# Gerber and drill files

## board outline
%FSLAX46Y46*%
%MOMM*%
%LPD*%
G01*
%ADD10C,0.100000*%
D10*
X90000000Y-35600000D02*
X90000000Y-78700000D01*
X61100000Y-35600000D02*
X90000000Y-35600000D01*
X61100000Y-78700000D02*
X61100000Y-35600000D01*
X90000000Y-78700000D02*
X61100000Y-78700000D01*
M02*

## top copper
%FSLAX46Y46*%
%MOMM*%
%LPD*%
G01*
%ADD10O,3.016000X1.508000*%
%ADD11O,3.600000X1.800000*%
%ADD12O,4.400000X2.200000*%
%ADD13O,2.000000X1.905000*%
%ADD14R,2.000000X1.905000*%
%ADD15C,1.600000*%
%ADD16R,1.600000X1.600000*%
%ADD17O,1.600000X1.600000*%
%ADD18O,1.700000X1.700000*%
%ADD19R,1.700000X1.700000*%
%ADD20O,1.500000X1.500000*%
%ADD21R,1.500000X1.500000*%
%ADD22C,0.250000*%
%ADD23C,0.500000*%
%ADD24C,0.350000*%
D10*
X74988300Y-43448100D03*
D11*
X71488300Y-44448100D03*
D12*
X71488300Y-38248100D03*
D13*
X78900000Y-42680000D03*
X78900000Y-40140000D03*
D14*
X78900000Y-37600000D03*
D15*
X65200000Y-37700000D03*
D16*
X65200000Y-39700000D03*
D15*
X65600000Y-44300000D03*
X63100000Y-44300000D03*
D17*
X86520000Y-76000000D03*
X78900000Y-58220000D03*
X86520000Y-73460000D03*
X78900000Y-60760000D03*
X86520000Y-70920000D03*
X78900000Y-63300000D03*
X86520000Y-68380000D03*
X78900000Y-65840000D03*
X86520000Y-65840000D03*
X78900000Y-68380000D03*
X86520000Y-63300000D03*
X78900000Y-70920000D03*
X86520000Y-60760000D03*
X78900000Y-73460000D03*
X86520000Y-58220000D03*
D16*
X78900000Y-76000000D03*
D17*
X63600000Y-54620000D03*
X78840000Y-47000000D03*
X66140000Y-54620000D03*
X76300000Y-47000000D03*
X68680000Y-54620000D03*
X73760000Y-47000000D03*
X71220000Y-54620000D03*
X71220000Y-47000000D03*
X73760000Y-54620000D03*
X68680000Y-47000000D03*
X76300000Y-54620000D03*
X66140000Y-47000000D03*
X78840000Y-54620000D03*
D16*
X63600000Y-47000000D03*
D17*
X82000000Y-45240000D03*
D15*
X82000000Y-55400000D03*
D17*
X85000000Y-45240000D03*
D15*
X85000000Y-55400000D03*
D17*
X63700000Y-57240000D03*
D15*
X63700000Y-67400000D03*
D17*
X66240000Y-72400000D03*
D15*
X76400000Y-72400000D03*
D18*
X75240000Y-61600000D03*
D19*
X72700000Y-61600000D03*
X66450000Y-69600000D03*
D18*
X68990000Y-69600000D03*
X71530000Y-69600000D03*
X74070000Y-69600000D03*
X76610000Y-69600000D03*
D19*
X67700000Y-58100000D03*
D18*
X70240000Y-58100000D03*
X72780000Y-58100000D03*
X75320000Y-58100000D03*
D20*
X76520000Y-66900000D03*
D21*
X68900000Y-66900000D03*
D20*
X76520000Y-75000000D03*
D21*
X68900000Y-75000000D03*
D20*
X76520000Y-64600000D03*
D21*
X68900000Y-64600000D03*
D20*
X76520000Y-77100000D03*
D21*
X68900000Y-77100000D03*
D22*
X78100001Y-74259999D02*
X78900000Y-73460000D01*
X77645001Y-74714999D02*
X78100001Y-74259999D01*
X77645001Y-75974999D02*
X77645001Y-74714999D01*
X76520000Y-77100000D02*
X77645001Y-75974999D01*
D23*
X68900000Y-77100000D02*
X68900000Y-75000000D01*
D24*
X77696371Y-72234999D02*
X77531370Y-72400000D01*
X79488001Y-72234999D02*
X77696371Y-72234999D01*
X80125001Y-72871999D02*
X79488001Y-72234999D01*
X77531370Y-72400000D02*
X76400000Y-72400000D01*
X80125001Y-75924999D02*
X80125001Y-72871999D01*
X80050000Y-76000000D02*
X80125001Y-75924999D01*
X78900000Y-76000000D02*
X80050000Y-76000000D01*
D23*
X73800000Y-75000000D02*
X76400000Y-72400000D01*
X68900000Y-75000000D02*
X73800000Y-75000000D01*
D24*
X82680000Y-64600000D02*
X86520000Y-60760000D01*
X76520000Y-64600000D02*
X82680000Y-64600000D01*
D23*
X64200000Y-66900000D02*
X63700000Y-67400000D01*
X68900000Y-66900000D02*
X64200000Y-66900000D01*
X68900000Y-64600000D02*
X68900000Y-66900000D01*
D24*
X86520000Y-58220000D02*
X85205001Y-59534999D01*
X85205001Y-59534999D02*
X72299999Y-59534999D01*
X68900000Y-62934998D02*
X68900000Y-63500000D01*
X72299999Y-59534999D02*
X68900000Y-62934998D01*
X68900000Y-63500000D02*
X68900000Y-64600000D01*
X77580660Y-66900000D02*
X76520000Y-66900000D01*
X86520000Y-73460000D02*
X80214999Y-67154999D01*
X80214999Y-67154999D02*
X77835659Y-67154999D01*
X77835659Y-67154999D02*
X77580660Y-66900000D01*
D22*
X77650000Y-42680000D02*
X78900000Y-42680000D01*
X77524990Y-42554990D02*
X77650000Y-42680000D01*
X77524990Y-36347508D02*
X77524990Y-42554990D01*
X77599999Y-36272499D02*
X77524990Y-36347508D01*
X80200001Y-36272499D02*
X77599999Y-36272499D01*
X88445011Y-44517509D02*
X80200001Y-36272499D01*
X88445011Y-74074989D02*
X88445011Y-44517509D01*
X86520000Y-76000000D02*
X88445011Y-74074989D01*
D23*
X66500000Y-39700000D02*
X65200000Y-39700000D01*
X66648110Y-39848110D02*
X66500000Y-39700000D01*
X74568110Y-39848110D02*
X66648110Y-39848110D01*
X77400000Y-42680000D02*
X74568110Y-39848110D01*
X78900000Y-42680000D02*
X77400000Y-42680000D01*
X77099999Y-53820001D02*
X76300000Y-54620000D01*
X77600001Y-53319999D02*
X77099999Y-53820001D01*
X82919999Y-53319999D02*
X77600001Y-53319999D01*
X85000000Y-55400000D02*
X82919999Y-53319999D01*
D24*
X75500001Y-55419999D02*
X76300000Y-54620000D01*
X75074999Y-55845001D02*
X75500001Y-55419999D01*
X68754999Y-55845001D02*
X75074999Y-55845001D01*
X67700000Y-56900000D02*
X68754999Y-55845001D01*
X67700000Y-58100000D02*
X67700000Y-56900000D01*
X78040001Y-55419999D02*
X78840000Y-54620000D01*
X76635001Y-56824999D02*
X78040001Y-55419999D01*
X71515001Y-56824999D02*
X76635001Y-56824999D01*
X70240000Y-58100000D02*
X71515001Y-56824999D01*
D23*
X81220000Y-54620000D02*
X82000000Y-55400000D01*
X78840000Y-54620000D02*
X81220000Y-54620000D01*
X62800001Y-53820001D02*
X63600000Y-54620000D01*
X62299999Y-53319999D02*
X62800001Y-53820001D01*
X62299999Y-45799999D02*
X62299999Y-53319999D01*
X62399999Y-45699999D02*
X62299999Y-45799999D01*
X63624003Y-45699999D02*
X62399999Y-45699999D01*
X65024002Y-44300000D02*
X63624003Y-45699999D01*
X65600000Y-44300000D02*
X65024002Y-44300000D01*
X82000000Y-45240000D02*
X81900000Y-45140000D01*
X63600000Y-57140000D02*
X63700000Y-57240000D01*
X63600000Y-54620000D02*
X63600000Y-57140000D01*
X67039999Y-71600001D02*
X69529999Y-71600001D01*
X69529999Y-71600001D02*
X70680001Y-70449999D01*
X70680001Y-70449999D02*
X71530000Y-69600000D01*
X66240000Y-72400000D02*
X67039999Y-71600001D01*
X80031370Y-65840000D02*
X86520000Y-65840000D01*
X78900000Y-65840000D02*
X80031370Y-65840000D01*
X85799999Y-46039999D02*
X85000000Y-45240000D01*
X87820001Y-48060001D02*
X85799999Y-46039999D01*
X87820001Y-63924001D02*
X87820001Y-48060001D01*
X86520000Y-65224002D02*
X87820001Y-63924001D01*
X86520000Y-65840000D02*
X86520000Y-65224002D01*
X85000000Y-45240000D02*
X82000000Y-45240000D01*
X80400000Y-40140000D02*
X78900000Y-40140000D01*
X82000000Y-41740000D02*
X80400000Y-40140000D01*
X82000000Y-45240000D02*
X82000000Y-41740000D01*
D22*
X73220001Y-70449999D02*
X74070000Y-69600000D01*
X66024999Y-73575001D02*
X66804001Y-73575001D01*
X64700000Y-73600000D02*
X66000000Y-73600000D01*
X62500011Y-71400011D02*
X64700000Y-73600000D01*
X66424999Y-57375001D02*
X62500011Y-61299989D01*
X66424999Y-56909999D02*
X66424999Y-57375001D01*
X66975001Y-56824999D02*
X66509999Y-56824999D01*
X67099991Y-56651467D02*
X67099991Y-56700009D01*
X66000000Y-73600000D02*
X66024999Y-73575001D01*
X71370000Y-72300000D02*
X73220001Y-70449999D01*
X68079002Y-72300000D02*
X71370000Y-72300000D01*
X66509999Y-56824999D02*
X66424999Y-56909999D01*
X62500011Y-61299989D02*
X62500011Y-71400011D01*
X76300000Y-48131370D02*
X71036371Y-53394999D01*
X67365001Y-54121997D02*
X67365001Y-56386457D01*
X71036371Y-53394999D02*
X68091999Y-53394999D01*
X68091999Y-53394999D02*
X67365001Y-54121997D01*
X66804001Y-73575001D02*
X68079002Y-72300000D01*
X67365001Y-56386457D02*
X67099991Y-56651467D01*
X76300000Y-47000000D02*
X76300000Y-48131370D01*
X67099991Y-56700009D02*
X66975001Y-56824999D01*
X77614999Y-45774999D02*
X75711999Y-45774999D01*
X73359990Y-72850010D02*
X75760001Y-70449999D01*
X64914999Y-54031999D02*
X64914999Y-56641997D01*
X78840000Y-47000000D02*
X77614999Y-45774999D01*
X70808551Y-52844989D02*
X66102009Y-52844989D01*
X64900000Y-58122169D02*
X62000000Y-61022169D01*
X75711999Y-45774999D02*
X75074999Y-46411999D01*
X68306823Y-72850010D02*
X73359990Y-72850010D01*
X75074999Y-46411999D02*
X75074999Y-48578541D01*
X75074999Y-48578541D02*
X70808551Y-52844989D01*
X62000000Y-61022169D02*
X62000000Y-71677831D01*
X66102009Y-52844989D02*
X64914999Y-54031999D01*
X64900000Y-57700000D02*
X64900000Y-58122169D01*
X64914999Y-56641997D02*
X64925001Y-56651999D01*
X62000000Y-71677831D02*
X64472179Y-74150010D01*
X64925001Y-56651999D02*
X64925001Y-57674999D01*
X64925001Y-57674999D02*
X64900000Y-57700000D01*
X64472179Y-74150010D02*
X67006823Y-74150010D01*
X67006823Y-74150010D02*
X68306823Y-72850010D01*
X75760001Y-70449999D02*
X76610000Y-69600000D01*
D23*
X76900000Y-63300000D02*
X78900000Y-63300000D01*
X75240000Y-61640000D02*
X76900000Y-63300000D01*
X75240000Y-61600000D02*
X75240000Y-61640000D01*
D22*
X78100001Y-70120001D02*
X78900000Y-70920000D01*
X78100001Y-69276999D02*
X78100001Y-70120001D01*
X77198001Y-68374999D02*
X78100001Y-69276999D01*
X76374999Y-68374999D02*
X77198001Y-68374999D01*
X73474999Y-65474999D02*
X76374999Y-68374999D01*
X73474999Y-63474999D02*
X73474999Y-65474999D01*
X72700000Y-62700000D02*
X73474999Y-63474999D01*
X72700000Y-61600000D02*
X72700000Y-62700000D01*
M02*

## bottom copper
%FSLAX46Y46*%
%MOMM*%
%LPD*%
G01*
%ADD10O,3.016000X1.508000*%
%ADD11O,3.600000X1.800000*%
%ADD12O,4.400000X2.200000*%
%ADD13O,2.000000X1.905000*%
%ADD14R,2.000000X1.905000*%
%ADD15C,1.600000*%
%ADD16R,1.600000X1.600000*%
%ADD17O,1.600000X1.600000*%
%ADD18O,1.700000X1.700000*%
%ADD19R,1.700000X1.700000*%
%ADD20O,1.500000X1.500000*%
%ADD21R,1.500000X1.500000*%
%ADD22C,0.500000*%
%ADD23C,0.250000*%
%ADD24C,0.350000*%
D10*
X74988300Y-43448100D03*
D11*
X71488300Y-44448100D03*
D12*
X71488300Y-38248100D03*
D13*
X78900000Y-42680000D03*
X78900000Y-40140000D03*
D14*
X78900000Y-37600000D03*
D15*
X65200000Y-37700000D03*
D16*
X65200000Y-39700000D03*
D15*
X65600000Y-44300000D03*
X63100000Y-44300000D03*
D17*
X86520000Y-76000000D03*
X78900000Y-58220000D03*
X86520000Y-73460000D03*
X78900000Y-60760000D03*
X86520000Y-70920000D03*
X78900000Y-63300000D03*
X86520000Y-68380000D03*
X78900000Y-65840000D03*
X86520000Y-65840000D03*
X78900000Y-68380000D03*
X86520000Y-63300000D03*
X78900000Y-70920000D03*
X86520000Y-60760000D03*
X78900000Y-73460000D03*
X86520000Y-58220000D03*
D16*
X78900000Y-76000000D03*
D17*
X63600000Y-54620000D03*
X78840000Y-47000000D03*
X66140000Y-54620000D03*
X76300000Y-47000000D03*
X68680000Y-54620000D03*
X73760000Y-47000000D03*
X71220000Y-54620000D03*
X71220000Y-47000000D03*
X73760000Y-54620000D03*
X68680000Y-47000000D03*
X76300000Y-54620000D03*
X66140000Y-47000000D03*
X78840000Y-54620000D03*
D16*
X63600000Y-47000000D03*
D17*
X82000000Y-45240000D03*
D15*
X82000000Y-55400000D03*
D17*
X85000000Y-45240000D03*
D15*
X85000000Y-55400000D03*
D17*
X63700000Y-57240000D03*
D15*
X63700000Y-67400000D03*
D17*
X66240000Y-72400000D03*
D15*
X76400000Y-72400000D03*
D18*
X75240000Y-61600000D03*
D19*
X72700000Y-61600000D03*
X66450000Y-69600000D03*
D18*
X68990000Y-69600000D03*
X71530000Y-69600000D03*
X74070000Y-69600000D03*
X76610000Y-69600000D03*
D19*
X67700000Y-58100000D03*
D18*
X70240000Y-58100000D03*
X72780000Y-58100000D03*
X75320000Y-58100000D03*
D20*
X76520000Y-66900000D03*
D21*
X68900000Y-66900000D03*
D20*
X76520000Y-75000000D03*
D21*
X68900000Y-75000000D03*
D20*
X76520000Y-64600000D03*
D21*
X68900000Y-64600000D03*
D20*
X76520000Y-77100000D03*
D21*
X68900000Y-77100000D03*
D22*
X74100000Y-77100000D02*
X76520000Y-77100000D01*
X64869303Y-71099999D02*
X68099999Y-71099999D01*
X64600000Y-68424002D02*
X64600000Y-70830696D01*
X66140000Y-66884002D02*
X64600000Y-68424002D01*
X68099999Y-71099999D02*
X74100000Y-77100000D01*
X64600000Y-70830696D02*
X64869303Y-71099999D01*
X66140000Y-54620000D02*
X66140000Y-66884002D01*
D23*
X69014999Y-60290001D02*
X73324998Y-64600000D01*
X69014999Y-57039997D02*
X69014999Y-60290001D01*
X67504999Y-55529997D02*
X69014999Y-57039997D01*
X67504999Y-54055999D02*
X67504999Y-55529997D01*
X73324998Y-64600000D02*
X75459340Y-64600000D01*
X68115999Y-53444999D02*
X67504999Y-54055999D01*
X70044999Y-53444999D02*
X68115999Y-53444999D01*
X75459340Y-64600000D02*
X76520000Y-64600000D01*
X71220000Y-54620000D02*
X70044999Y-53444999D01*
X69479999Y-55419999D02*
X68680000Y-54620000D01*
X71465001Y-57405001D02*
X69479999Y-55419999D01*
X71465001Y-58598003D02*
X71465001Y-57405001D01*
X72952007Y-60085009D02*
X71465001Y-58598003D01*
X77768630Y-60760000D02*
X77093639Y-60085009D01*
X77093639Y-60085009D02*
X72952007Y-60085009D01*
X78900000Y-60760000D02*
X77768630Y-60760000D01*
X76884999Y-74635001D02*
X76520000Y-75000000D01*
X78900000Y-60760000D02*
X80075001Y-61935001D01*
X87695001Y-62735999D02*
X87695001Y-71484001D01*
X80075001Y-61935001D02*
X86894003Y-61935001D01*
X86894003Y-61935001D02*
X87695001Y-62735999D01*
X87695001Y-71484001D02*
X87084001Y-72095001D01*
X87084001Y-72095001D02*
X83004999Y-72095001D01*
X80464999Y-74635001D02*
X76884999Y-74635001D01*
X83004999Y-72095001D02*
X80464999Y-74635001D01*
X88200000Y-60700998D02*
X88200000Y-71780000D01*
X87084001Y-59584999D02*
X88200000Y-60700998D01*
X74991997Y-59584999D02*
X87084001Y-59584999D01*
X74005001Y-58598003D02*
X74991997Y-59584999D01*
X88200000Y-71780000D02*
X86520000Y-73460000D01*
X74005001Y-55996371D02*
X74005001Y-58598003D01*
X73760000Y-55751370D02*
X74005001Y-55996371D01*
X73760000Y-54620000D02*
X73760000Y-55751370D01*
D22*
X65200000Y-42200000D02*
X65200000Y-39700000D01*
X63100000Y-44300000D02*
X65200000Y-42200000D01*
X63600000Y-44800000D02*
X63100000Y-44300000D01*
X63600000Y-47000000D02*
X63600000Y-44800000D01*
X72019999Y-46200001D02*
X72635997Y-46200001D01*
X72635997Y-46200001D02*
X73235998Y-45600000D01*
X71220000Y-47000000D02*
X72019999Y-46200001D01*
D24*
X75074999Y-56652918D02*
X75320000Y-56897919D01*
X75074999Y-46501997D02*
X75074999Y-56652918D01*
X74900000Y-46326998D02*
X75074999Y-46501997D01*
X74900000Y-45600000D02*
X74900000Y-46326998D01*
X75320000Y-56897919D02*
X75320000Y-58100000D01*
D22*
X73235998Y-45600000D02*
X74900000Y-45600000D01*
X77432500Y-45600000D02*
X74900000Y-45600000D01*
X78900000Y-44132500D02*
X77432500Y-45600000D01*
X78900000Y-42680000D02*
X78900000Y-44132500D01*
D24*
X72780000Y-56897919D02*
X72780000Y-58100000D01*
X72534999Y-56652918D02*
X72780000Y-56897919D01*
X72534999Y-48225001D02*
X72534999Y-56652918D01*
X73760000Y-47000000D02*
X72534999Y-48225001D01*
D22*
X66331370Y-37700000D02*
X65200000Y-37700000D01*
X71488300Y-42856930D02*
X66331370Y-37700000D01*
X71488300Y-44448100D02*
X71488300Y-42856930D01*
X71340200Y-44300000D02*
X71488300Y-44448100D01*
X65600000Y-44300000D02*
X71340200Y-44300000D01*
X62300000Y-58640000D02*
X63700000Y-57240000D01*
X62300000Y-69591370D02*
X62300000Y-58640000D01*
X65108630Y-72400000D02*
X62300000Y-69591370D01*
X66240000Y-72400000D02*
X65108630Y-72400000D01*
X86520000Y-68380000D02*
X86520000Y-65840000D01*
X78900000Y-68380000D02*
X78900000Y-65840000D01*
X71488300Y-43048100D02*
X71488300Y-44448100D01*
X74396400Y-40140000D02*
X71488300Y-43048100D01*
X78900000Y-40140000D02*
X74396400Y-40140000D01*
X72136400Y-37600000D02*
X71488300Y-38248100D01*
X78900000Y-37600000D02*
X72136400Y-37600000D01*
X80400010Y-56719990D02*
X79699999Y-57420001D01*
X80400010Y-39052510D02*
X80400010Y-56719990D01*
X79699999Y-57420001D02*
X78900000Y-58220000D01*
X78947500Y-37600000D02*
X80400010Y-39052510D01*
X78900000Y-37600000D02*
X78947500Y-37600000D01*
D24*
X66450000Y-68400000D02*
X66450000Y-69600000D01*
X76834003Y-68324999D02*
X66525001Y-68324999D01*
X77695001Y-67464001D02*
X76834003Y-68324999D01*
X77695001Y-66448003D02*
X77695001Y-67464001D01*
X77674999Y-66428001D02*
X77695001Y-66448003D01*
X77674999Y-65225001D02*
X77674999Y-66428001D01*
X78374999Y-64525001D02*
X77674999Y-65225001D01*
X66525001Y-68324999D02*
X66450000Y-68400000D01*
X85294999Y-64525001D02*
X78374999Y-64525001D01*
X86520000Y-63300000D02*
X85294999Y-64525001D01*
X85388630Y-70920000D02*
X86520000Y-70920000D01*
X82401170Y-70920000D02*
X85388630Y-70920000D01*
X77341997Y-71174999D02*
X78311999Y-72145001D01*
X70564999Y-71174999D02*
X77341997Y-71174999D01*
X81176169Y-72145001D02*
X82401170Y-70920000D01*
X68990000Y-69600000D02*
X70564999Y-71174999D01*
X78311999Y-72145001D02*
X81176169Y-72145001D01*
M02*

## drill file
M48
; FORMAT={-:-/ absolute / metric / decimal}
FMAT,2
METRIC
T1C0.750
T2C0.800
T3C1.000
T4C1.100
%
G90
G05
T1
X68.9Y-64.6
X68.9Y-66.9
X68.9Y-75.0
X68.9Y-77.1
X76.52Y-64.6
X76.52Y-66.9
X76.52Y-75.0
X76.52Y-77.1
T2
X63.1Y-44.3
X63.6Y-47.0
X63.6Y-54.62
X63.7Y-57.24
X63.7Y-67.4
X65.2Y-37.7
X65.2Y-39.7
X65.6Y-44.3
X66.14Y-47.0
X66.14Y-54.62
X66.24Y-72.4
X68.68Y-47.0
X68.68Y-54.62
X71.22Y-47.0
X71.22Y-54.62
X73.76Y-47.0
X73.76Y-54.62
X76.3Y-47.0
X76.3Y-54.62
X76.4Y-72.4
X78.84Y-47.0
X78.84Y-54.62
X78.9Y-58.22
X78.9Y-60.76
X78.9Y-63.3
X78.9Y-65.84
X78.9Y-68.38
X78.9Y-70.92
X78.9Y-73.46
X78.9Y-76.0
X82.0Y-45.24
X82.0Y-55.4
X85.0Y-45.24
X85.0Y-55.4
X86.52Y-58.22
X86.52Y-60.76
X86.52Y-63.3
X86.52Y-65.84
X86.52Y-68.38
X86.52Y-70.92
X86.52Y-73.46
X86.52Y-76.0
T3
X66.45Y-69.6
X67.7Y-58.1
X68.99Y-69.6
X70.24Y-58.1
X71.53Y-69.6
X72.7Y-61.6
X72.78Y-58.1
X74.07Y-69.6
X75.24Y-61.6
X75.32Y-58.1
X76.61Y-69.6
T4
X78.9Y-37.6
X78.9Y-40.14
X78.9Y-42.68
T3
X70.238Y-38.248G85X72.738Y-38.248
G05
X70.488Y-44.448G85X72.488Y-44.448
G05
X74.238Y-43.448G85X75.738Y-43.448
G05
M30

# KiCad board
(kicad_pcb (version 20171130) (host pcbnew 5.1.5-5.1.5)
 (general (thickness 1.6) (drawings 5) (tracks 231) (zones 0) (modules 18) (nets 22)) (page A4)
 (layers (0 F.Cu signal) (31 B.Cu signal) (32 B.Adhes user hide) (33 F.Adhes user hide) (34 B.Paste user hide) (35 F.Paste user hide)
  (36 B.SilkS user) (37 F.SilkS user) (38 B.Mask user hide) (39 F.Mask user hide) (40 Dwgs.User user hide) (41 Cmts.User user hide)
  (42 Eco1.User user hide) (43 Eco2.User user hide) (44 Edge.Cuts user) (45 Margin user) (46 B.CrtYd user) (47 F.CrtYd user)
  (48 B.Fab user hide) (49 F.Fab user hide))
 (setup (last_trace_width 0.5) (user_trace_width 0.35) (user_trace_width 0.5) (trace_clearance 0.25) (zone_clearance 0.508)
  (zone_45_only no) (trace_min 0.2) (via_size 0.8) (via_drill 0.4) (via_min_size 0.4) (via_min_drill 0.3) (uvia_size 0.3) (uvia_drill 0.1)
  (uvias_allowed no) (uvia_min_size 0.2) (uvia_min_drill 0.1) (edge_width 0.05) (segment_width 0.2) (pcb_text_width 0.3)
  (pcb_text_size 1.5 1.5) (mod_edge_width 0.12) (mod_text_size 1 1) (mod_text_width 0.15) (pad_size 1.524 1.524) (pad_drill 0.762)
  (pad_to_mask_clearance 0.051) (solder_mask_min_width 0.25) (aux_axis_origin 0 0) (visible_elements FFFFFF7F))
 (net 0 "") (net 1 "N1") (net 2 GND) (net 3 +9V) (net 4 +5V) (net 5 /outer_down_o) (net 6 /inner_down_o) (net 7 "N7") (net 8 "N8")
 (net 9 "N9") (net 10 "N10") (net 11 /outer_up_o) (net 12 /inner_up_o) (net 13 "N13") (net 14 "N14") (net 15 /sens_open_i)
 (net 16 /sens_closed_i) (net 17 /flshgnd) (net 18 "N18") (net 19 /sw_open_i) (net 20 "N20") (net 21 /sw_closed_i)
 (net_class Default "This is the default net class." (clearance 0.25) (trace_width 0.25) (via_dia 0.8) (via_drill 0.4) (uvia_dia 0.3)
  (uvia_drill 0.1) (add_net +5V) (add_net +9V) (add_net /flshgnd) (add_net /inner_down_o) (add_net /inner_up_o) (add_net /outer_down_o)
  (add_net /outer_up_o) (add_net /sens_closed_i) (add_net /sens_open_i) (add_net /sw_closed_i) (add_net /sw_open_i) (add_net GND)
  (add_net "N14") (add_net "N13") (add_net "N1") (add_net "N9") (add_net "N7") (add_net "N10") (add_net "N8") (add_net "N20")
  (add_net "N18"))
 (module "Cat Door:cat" (layer B.Cu) (at 85.2 39.8 180)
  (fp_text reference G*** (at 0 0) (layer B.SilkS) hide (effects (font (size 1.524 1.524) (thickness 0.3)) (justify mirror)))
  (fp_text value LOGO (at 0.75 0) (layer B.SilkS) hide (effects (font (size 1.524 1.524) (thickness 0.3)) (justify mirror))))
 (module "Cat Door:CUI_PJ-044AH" (layer F.Cu) (at 71.4883 41.9481)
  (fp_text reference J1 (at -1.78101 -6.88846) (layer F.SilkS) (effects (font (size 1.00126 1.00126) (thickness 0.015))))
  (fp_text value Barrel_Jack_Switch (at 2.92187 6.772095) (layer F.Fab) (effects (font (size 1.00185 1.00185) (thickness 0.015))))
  (pad 3 thru_hole oval (at 3.5 1.5) (size 3.016 1.508) (drill oval 2.5 1) (layers *.Cu *.Mask) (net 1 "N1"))
  (pad 2 thru_hole oval (at 0 2.5) (size 3.6 1.8) (drill oval 3 1) (layers *.Cu *.Mask) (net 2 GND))
  (pad 1 thru_hole oval (at 0 -3.7) (size 4.4 2.2) (drill oval 3.5 1) (layers *.Cu *.Mask) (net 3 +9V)))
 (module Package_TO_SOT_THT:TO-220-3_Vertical (layer B.Cu) (at 78.9 37.6 270)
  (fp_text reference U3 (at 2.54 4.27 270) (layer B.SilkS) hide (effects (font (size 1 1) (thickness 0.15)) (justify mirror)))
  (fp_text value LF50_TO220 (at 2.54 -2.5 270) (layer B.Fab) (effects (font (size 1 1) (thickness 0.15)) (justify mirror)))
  (pad 3 thru_hole oval (at 5.08 0 270) (size 1.905 2) (drill 1.1) (layers *.Cu *.Mask) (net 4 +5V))
  (pad 2 thru_hole oval (at 2.54 0 270) (size 1.905 2) (drill 1.1) (layers *.Cu *.Mask) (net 2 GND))
  (pad 1 thru_hole rect (at 0 0 270) (size 1.905 2) (drill 1.1) (layers *.Cu *.Mask) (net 3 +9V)))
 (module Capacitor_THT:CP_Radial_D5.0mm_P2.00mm (layer B.Cu) (at 65.2 39.7 90)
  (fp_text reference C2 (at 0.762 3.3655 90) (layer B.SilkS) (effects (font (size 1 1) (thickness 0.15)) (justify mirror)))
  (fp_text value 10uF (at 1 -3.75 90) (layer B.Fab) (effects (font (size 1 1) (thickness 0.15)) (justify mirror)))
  (pad 2 thru_hole circle (at 2 0 90) (size 1.6 1.6) (drill 0.8) (layers *.Cu *.Mask) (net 2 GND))
  (pad 1 thru_hole rect (at 0 0 90) (size 1.6 1.6) (drill 0.8) (layers *.Cu *.Mask) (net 4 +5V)))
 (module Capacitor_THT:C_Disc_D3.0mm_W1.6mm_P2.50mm (layer B.Cu) (at 63.1 44.3)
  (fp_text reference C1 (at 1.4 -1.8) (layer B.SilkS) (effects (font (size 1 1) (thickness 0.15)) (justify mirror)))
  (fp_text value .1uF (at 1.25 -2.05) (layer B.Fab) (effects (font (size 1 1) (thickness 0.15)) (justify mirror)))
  (pad 2 thru_hole circle (at 2.5 0) (size 1.6 1.6) (drill 0.8) (layers *.Cu *.Mask) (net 2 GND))
  (pad 1 thru_hole circle (at 0 0) (size 1.6 1.6) (drill 0.8) (layers *.Cu *.Mask) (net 4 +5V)))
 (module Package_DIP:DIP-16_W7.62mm (layer B.Cu) (at 78.9 76)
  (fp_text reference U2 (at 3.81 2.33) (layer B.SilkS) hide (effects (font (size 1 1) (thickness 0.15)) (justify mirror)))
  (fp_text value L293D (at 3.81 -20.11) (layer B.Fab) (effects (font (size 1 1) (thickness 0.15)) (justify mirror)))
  (pad 16 thru_hole oval (at 7.62 0) (size 1.6 1.6) (drill 0.8) (layers *.Cu *.Mask) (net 4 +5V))
  (pad 8 thru_hole oval (at 0 -17.78) (size 1.6 1.6) (drill 0.8) (layers *.Cu *.Mask) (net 3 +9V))
  (pad 15 thru_hole oval (at 7.62 -2.54) (size 1.6 1.6) (drill 0.8) (layers *.Cu *.Mask) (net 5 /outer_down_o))
  (pad 7 thru_hole oval (at 0 -15.24) (size 1.6 1.6) (drill 0.8) (layers *.Cu *.Mask) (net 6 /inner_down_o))
  (pad 14 thru_hole oval (at 7.62 -5.08) (size 1.6 1.6) (drill 0.8) (layers *.Cu *.Mask) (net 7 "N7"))
  (pad 6 thru_hole oval (at 0 -12.7) (size 1.6 1.6) (drill 0.8) (layers *.Cu *.Mask) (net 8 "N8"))
  (pad 13 thru_hole oval (at 7.62 -7.62) (size 1.6 1.6) (drill 0.8) (layers *.Cu *.Mask) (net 2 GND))
  (pad 5 thru_hole oval (at 0 -10.16) (size 1.6 1.6) (drill 0.8) (layers *.Cu *.Mask) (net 2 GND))
  (pad 12 thru_hole oval (at 7.62 -10.16) (size 1.6 1.6) (drill 0.8) (layers *.Cu *.Mask) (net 2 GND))
  (pad 4 thru_hole oval (at 0 -7.62) (size 1.6 1.6) (drill 0.8) (layers *.Cu *.Mask) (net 2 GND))
  (pad 11 thru_hole oval (at 7.62 -12.7) (size 1.6 1.6) (drill 0.8) (layers *.Cu *.Mask) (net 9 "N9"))
  (pad 3 thru_hole oval (at 0 -5.08) (size 1.6 1.6) (drill 0.8) (layers *.Cu *.Mask) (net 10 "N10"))
  (pad 10 thru_hole oval (at 7.62 -15.24) (size 1.6 1.6) (drill 0.8) (layers *.Cu *.Mask) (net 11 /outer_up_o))
  (pad 2 thru_hole oval (at 0 -2.54) (size 1.6 1.6) (drill 0.8) (layers *.Cu *.Mask) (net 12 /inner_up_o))
  (pad 9 thru_hole oval (at 7.62 -17.78) (size 1.6 1.6) (drill 0.8) (layers *.Cu *.Mask) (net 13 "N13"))
  (pad 1 thru_hole rect (at 0 0) (size 1.6 1.6) (drill 0.8) (layers *.Cu *.Mask) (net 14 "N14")))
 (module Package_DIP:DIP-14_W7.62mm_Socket (layer B.Cu) (at 63.6 47 270)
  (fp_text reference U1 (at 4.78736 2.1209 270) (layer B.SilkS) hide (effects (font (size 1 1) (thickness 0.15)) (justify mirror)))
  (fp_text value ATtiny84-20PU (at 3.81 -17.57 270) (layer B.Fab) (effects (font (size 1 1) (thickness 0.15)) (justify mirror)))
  (pad 14 thru_hole oval (at 7.62 0 270) (size 1.6 1.6) (drill 0.8) (layers *.Cu *.Mask) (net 2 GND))
  (pad 7 thru_hole oval (at 0 -15.24 270) (size 1.6 1.6) (drill 0.8) (layers *.Cu *.Mask) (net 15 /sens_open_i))
  (pad 13 thru_hole oval (at 7.62 -2.54 270) (size 1.6 1.6) (drill 0.8) (layers *.Cu *.Mask) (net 12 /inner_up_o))
  (pad 6 thru_hole oval (at 0 -12.7 270) (size 1.6 1.6) (drill 0.8) (layers *.Cu *.Mask) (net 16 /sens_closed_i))
  (pad 12 thru_hole oval (at 7.62 -5.08 270) (size 1.6 1.6) (drill 0.8) (layers *.Cu *.Mask) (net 6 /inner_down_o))
  (pad 5 thru_hole oval (at 0 -10.16 270) (size 1.6 1.6) (drill 0.8) (layers *.Cu *.Mask) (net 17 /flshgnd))
  (pad 11 thru_hole oval (at 7.62 -7.62 270) (size 1.6 1.6) (drill 0.8) (layers *.Cu *.Mask) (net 11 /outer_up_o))
  (pad 4 thru_hole oval (at 0 -7.62 270) (size 1.6 1.6) (drill 0.8) (layers *.Cu *.Mask) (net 4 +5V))
  (pad 10 thru_hole oval (at 7.62 -10.16 270) (size 1.6 1.6) (drill 0.8) (layers *.Cu *.Mask) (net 5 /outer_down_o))
  (pad 3 thru_hole oval (at 0 -5.08 270) (size 1.6 1.6) (drill 0.8) (layers *.Cu *.Mask) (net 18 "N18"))
  (pad 9 thru_hole oval (at 7.62 -12.7 270) (size 1.6 1.6) (drill 0.8) (layers *.Cu *.Mask) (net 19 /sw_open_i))
  (pad 2 thru_hole oval (at 0 -2.54 270) (size 1.6 1.6) (drill 0.8) (layers *.Cu *.Mask) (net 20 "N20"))
  (pad 8 thru_hole oval (at 7.62 -15.24 270) (size 1.6 1.6) (drill 0.8) (layers *.Cu *.Mask) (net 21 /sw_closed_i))
  (pad 1 thru_hole rect (at 0 0 270) (size 1.6 1.6) (drill 0.8) (layers *.Cu *.Mask) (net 4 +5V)))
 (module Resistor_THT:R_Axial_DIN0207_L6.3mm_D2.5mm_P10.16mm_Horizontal (layer B.Cu) (at 82 55.4 90)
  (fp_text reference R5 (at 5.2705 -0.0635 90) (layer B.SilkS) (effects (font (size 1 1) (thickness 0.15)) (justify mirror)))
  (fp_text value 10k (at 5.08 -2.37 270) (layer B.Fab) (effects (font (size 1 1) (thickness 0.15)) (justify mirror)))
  (pad 2 thru_hole oval (at 10.16 0 90) (size 1.6 1.6) (drill 0.8) (layers *.Cu *.Mask) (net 2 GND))
  (pad 1 thru_hole circle (at 0 0 90) (size 1.6 1.6) (drill 0.8) (layers *.Cu *.Mask) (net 21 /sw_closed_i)))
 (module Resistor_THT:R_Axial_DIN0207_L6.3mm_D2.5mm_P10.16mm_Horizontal (layer B.Cu) (at 85 55.4 90)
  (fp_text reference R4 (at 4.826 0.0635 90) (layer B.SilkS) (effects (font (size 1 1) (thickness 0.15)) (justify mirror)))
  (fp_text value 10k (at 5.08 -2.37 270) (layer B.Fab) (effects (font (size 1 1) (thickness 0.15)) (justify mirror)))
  (pad 2 thru_hole oval (at 10.16 0 90) (size 1.6 1.6) (drill 0.8) (layers *.Cu *.Mask) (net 2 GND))
  (pad 1 thru_hole circle (at 0 0 90) (size 1.6 1.6) (drill 0.8) (layers *.Cu *.Mask) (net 19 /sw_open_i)))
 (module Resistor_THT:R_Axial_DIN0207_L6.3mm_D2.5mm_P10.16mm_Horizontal (layer B.Cu) (at 63.7 67.4 90)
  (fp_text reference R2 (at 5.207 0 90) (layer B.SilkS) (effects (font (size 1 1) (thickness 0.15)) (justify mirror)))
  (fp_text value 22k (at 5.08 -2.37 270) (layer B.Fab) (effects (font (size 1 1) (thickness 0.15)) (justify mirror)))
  (pad 2 thru_hole oval (at 10.16 0 90) (size 1.6 1.6) (drill 0.8) (layers *.Cu *.Mask) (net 2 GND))
  (pad 1 thru_hole circle (at 0 0 90) (size 1.6 1.6) (drill 0.8) (layers *.Cu *.Mask) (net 13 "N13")))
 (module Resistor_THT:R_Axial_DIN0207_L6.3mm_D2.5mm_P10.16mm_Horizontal (layer B.Cu) (at 76.4 72.4 180)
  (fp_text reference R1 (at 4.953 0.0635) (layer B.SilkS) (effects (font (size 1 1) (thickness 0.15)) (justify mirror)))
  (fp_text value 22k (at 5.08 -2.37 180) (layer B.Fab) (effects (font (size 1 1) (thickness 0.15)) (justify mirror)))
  (pad 2 thru_hole oval (at 10.16 0 180) (size 1.6 1.6) (drill 0.8) (layers *.Cu *.Mask) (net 2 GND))
  (pad 1 thru_hole circle (at 0 0 180) (size 1.6 1.6) (drill 0.8) (layers *.Cu *.Mask) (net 14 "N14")))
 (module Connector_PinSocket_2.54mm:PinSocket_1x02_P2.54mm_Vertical (layer B.Cu) (at 72.7 61.6 270)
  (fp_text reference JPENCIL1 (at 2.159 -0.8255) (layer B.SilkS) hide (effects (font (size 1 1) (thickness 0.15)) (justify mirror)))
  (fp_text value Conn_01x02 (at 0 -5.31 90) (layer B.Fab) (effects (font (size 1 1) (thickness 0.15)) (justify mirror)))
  (pad 2 thru_hole oval (at 0 -2.54 270) (size 1.7 1.7) (drill 1) (layers *.Cu *.Mask) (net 8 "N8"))
  (pad 1 thru_hole rect (at 0 0 270) (size 1.7 1.7) (drill 1) (layers *.Cu *.Mask) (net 10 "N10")))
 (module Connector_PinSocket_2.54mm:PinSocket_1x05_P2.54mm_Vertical (layer F.Cu) (at 66.45 69.6 90)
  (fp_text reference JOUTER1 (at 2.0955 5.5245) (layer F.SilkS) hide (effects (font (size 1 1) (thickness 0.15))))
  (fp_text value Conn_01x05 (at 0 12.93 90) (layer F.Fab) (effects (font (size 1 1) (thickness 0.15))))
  (pad 1 thru_hole rect (at 0 0 90) (size 1.7 1.7) (drill 1) (layers *.Cu *.Mask) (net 9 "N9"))
  (pad 2 thru_hole oval (at 0 2.54 90) (size 1.7 1.7) (drill 1) (layers *.Cu *.Mask) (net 7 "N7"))
  (pad 3 thru_hole oval (at 0 5.08 90) (size 1.7 1.7) (drill 1) (layers *.Cu *.Mask) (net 2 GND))
  (pad 4 thru_hole oval (at 0 7.62 90) (size 1.7 1.7) (drill 1) (layers *.Cu *.Mask) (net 16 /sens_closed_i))
  (pad 5 thru_hole oval (at 0 10.16 90) (size 1.7 1.7) (drill 1) (layers *.Cu *.Mask) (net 15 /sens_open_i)))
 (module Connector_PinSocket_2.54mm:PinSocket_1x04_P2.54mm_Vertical (layer F.Cu) (at 67.7 58.1 90)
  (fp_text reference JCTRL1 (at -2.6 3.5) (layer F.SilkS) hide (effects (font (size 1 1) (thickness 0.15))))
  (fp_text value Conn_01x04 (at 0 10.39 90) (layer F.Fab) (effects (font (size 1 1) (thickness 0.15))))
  (pad 1 thru_hole rect (at 0 0 90) (size 1.7 1.7) (drill 1) (layers *.Cu *.Mask) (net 19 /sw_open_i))
  (pad 2 thru_hole oval (at 0 2.54 90) (size 1.7 1.7) (drill 1) (layers *.Cu *.Mask) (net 21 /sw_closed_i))
  (pad 3 thru_hole oval (at 0 5.08 90) (size 1.7 1.7) (drill 1) (layers *.Cu *.Mask) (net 17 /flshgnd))
  (pad 4 thru_hole oval (at 0 7.62 90) (size 1.7 1.7) (drill 1) (layers *.Cu *.Mask) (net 4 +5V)))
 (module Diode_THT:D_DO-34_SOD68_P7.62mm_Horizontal (layer B.Cu) (at 68.9 66.9)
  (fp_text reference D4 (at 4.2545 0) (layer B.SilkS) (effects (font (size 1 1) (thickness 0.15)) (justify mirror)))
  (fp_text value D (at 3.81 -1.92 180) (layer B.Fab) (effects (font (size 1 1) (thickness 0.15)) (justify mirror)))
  (pad 2 thru_hole oval (at 7.62 0) (size 1.5 1.5) (drill 0.75) (layers *.Cu *.Mask) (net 5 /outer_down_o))
  (pad 1 thru_hole rect (at 0 0) (size 1.5 1.5) (drill 0.75) (layers *.Cu *.Mask) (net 13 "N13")))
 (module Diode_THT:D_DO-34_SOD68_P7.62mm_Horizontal (layer B.Cu) (at 68.9 75)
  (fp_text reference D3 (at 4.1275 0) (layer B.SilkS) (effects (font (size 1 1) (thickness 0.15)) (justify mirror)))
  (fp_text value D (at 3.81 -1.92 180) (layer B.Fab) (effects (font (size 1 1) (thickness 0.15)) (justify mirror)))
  (pad 2 thru_hole oval (at 7.62 0) (size 1.5 1.5) (drill 0.75) (layers *.Cu *.Mask) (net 6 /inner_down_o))
  (pad 1 thru_hole rect (at 0 0) (size 1.5 1.5) (drill 0.75) (layers *.Cu *.Mask) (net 14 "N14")))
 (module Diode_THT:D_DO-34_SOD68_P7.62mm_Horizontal (layer B.Cu) (at 68.9 64.6)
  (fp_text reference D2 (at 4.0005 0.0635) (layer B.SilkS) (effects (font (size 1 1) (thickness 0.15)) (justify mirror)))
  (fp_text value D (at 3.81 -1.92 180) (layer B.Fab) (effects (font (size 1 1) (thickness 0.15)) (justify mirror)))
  (pad 2 thru_hole oval (at 7.62 0) (size 1.5 1.5) (drill 0.75) (layers *.Cu *.Mask) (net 11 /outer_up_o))
  (pad 1 thru_hole rect (at 0 0) (size 1.5 1.5) (drill 0.75) (layers *.Cu *.Mask) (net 13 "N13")))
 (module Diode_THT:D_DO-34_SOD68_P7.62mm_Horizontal (layer B.Cu) (at 68.9 77.1)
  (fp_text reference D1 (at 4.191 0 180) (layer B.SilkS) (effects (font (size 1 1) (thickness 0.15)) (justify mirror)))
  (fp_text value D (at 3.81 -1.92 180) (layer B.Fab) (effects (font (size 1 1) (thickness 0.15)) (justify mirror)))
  (pad 2 thru_hole oval (at 7.62 0) (size 1.5 1.5) (drill 0.75) (layers *.Cu *.Mask) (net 12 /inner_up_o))
  (pad 1 thru_hole rect (at 0 0) (size 1.5 1.5) (drill 0.75) (layers *.Cu *.Mask) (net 14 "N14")))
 (gr_line (start 90 35.6) (end 90 78.7) (layer Edge.Cuts) (width 0.1))
 (gr_line (start 61.1 35.6) (end 90 35.6) (layer Edge.Cuts) (width 0.1))
 (gr_line (start 61.1 78.7) (end 61.1 35.6) (layer Edge.Cuts) (width 0.1))
 (gr_line (start 90 78.7) (end 61.1 78.7) (layer Edge.Cuts) (width 0.1))
 (segment (start 78.100001 74.259999) (end 78.9 73.46) (width 0.25) (layer F.Cu) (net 12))
 (segment (start 77.645001 74.714999) (end 78.100001 74.259999) (width 0.25) (layer F.Cu) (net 12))
 (segment (start 77.645001 75.974999) (end 77.645001 74.714999) (width 0.25) (layer F.Cu) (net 12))
 (segment (start 76.52 77.1) (end 77.645001 75.974999) (width 0.25) (layer F.Cu) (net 12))
 (segment (start 74.1 77.1) (end 76.52 77.1) (width 0.5) (layer B.Cu) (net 12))
 (segment (start 64.869303 71.099999) (end 68.099999 71.099999) (width 0.5) (layer B.Cu) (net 12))
 (segment (start 64.6 68.424002) (end 64.6 70.830696) (width 0.5) (layer B.Cu) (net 12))
 (segment (start 66.14 66.884002) (end 64.6 68.424002) (width 0.5) (layer B.Cu) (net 12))
 (segment (start 68.099999 71.099999) (end 74.1 77.1) (width 0.5) (layer B.Cu) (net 12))
 (segment (start 64.6 70.830696) (end 64.869303 71.099999) (width 0.5) (layer B.Cu) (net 12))
 (segment (start 66.14 54.62) (end 66.14 66.884002) (width 0.5) (layer B.Cu) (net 12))
 (segment (start 68.9 77.1) (end 68.9 75) (width 0.5) (layer F.Cu) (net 14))
 (segment (start 77.696371 72.234999) (end 77.53137 72.4) (width 0.35) (layer F.Cu) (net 14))
 (segment (start 79.488001 72.234999) (end 77.696371 72.234999) (width 0.35) (layer F.Cu) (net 14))
 (segment (start 80.125001 72.871999) (end 79.488001 72.234999) (width 0.35) (layer F.Cu) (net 14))
 (segment (start 77.53137 72.4) (end 76.4 72.4) (width 0.35) (layer F.Cu) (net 14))
 (segment (start 80.125001 75.924999) (end 80.125001 72.871999) (width 0.35) (layer F.Cu) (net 14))
 (segment (start 80.05 76) (end 80.125001 75.924999) (width 0.35) (layer F.Cu) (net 14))
 (segment (start 78.9 76) (end 80.05 76) (width 0.35) (layer F.Cu) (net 14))
 (segment (start 73.8 75) (end 76.4 72.4) (width 0.5) (layer F.Cu) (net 14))
 (segment (start 68.9 75) (end 73.8 75) (width 0.5) (layer F.Cu) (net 14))
 (segment (start 82.68 64.6) (end 86.52 60.76) (width 0.35) (layer F.Cu) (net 11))
 (segment (start 76.52 64.6) (end 82.68 64.6) (width 0.35) (layer F.Cu) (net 11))
 (segment (start 69.014999 60.290001) (end 73.324998 64.6) (width 0.25) (layer B.Cu) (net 11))
 (segment (start 69.014999 57.039997) (end 69.014999 60.290001) (width 0.25) (layer B.Cu) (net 11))
 (segment (start 67.504999 55.529997) (end 69.014999 57.039997) (width 0.25) (layer B.Cu) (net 11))
 (segment (start 67.504999 54.055999) (end 67.504999 55.529997) (width 0.25) (layer B.Cu) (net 11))
 (segment (start 73.324998 64.6) (end 75.45934 64.6) (width 0.25) (layer B.Cu) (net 11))
 (segment (start 68.115999 53.444999) (end 67.504999 54.055999) (width 0.25) (layer B.Cu) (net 11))
 (segment (start 70.044999 53.444999) (end 68.115999 53.444999) (width 0.25) (layer B.Cu) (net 11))
 (segment (start 75.45934 64.6) (end 76.52 64.6) (width 0.25) (layer B.Cu) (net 11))
 (segment (start 71.22 54.62) (end 70.044999 53.444999) (width 0.25) (layer B.Cu) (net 11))
 (segment (start 64.2 66.9) (end 63.7 67.4) (width 0.5) (layer F.Cu) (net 13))
 (segment (start 68.9 66.9) (end 64.2 66.9) (width 0.5) (layer F.Cu) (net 13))
 (segment (start 68.9 64.6) (end 68.9 66.9) (width 0.5) (layer F.Cu) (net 13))
 (segment (start 86.52 58.22) (end 85.205001 59.534999) (width 0.35) (layer F.Cu) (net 13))
 (segment (start 85.205001 59.534999) (end 72.299999 59.534999) (width 0.35) (layer F.Cu) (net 13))
 (segment (start 68.9 62.934998) (end 68.9 63.5) (width 0.35) (layer F.Cu) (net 13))
 (segment (start 72.299999 59.534999) (end 68.9 62.934998) (width 0.35) (layer F.Cu) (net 13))
 (segment (start 68.9 63.5) (end 68.9 64.6) (width 0.35) (layer F.Cu) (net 13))
 (segment (start 69.479999 55.419999) (end 68.68 54.62) (width 0.25) (layer B.Cu) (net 6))
 (segment (start 71.465001 57.405001) (end 69.479999 55.419999) (width 0.25) (layer B.Cu) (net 6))
 (segment (start 71.465001 58.598003) (end 71.465001 57.405001) (width 0.25) (layer B.Cu) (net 6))
 (segment (start 72.952007 60.085009) (end 71.465001 58.598003) (width 0.25) (layer B.Cu) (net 6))
 (segment (start 77.76863 60.76) (end 77.093639 60.085009) (width 0.25) (layer B.Cu) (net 6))
 (segment (start 77.093639 60.085009) (end 72.952007 60.085009) (width 0.25) (layer B.Cu) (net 6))
 (segment (start 78.9 60.76) (end 77.76863 60.76) (width 0.25) (layer B.Cu) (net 6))
 (segment (start 76.884999 74.635001) (end 76.52 75) (width 0.25) (layer B.Cu) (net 6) (status 1000000))
 (segment (start 78.9 60.76) (end 80.075001 61.935001) (width 0.25) (layer B.Cu) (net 6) (status 1000000))
 (segment (start 87.695001 62.735999) (end 87.695001 71.484001) (width 0.25) (layer B.Cu) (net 6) (status 1000000))
 (segment (start 80.075001 61.935001) (end 86.894003 61.935001) (width 0.25) (layer B.Cu) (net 6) (status 1000000))
 (segment (start 86.894003 61.935001) (end 87.695001 62.735999) (width 0.25) (layer B.Cu) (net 6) (status 1000000))
 (segment (start 87.695001 71.484001) (end 87.084001 72.095001) (width 0.25) (layer B.Cu) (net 6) (status 1000000))
 (segment (start 87.084001 72.095001) (end 83.004999 72.095001) (width 0.25) (layer B.Cu) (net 6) (status 1000000))
 (segment (start 80.464999 74.635001) (end 76.884999 74.635001) (width 0.25) (layer B.Cu) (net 6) (status 1000000))
 (segment (start 83.004999 72.095001) (end 80.464999 74.635001) (width 0.25) (layer B.Cu) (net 6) (status 1000000))
 (segment (start 77.58066 66.9) (end 76.52 66.9) (width 0.35) (layer F.Cu) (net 5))
 (segment (start 86.52 73.46) (end 80.214999 67.154999) (width 0.35) (layer F.Cu) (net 5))
 (segment (start 80.214999 67.154999) (end 77.835659 67.154999) (width 0.35) (layer F.Cu) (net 5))
 (segment (start 77.835659 67.154999) (end 77.58066 66.9) (width 0.35) (layer F.Cu) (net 5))
 (segment (start 88.2 60.700998) (end 88.2 71.78) (width 0.25) (layer B.Cu) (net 5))
 (segment (start 87.084001 59.584999) (end 88.2 60.700998) (width 0.25) (layer B.Cu) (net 5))
 (segment (start 74.991997 59.584999) (end 87.084001 59.584999) (width 0.25) (layer B.Cu) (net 5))
 (segment (start 74.005001 58.598003) (end 74.991997 59.584999) (width 0.25) (layer B.Cu) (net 5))
 (segment (start 88.2 71.78) (end 86.52 73.46) (width 0.25) (layer B.Cu) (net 5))
 (segment (start 74.005001 55.996371) (end 74.005001 58.598003) (width 0.25) (layer B.Cu) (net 5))
 (segment (start 73.76 55.75137) (end 74.005001 55.996371) (width 0.25) (layer B.Cu) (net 5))
 (segment (start 73.76 54.62) (end 73.76 55.75137) (width 0.25) (layer B.Cu) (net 5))
 (segment (start 65.2 42.2) (end 65.2 39.7) (width 0.5) (layer B.Cu) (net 4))
 (segment (start 63.1 44.3) (end 65.2 42.2) (width 0.5) (layer B.Cu) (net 4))
 (segment (start 63.6 44.8) (end 63.1 44.3) (width 0.5) (layer B.Cu) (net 4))
 (segment (start 63.6 47) (end 63.6 44.8) (width 0.5) (layer B.Cu) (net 4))
 (segment (start 72.019999 46.200001) (end 72.635997 46.200001) (width 0.5) (layer B.Cu) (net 4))
 (segment (start 72.635997 46.200001) (end 73.235998 45.6) (width 0.5) (layer B.Cu) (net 4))
 (segment (start 71.22 47) (end 72.019999 46.200001) (width 0.5) (layer B.Cu) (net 4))
 (segment (start 75.074999 56.652918) (end 75.32 56.897919) (width 0.35) (layer B.Cu) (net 4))
 (segment (start 75.074999 46.501997) (end 75.074999 56.652918) (width 0.35) (layer B.Cu) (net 4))
 (segment (start 74.9 46.326998) (end 75.074999 46.501997) (width 0.35) (layer B.Cu) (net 4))
 (segment (start 74.9 45.6) (end 74.9 46.326998) (width 0.35) (layer B.Cu) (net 4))
 (segment (start 75.32 56.897919) (end 75.32 58.1) (width 0.35) (layer B.Cu) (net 4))
 (segment (start 73.235998 45.6) (end 74.9 45.6) (width 0.5) (layer B.Cu) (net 4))
 (segment (start 77.65 42.68) (end 78.9 42.68) (width 0.25) (layer F.Cu) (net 4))
 (segment (start 77.52499 42.55499) (end 77.65 42.68) (width 0.25) (layer F.Cu) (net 4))
 (segment (start 77.52499 36.347508) (end 77.52499 42.55499) (width 0.25) (layer F.Cu) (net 4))
 (segment (start 77.599999 36.272499) (end 77.52499 36.347508) (width 0.25) (layer F.Cu) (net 4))
 (segment (start 80.200001 36.272499) (end 77.599999 36.272499) (width 0.25) (layer F.Cu) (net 4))
 (segment (start 88.445011 44.517509) (end 80.200001 36.272499) (width 0.25) (layer F.Cu) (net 4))
 (segment (start 88.445011 74.074989) (end 88.445011 44.517509) (width 0.25) (layer F.Cu) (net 4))
 (segment (start 86.52 76) (end 88.445011 74.074989) (width 0.25) (layer F.Cu) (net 4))
 (segment (start 77.4325 45.6) (end 74.9 45.6) (width 0.5) (layer B.Cu) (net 4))
 (segment (start 78.9 44.1325) (end 77.4325 45.6) (width 0.5) (layer B.Cu) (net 4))
 (segment (start 78.9 42.68) (end 78.9 44.1325) (width 0.5) (layer B.Cu) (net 4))
 (segment (start 66.5 39.7) (end 65.2 39.7) (width 0.5) (layer F.Cu) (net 4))
 (segment (start 66.64811 39.84811) (end 66.5 39.7) (width 0.5) (layer F.Cu) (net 4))
 (segment (start 74.56811 39.84811) (end 66.64811 39.84811) (width 0.5) (layer F.Cu) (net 4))
 (segment (start 77.4 42.68) (end 74.56811 39.84811) (width 0.5) (layer F.Cu) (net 4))
 (segment (start 78.9 42.68) (end 77.4 42.68) (width 0.5) (layer F.Cu) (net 4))
 (segment (start 72.78 56.897919) (end 72.78 58.1) (width 0.35) (layer B.Cu) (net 17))
 (segment (start 72.534999 56.652918) (end 72.78 56.897919) (width 0.35) (layer B.Cu) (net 17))
 (segment (start 72.534999 48.225001) (end 72.534999 56.652918) (width 0.35) (layer B.Cu) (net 17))
 (segment (start 73.76 47) (end 72.534999 48.225001) (width 0.35) (layer B.Cu) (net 17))
 (segment (start 77.099999 53.820001) (end 76.3 54.62) (width 0.5) (layer F.Cu) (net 19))
 (segment (start 77.600001 53.319999) (end 77.099999 53.820001) (width 0.5) (layer F.Cu) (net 19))
 (segment (start 82.919999 53.319999) (end 77.600001 53.319999) (width 0.5) (layer F.Cu) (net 19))
 (segment (start 85 55.4) (end 82.919999 53.319999) (width 0.5) (layer F.Cu) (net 19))
 (segment (start 75.500001 55.419999) (end 76.3 54.62) (width 0.35) (layer F.Cu) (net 19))
 (segment (start 75.074999 55.845001) (end 75.500001 55.419999) (width 0.35) (layer F.Cu) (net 19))
 (segment (start 68.754999 55.845001) (end 75.074999 55.845001) (width 0.35) (layer F.Cu) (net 19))
 (segment (start 67.7 56.9) (end 68.754999 55.845001) (width 0.35) (layer F.Cu) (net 19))
 (segment (start 67.7 58.1) (end 67.7 56.9) (width 0.35) (layer F.Cu) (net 19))
 (segment (start 78.040001 55.419999) (end 78.84 54.62) (width 0.35) (layer F.Cu) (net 21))
 (segment (start 76.635001 56.824999) (end 78.040001 55.419999) (width 0.35) (layer F.Cu) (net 21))
 (segment (start 71.515001 56.824999) (end 76.635001 56.824999) (width 0.35) (layer F.Cu) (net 21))
 (segment (start 70.24 58.1) (end 71.515001 56.824999) (width 0.35) (layer F.Cu) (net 21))
 (segment (start 81.22 54.62) (end 82 55.4) (width 0.5) (layer F.Cu) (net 21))
 (segment (start 78.84 54.62) (end 81.22 54.62) (width 0.5) (layer F.Cu) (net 21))
 (segment (start 66.33137 37.7) (end 65.2 37.7) (width 0.5) (layer B.Cu) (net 2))
 (segment (start 71.4883 42.85693) (end 66.33137 37.7) (width 0.5) (layer B.Cu) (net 2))
 (segment (start 71.4883 44.4481) (end 71.4883 42.85693) (width 0.5) (layer B.Cu) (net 2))
 (segment (start 71.3402 44.3) (end 71.4883 44.4481) (width 0.5) (layer B.Cu) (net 2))
 (segment (start 65.6 44.3) (end 71.3402 44.3) (width 0.5) (layer B.Cu) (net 2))
 (segment (start 62.800001 53.820001) (end 63.6 54.62) (width 0.5) (layer F.Cu) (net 2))
 (segment (start 62.299999 53.319999) (end 62.800001 53.820001) (width 0.5) (layer F.Cu) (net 2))
 (segment (start 62.299999 45.799999) (end 62.299999 53.319999) (width 0.5) (layer F.Cu) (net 2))
 (segment (start 62.399999 45.699999) (end 62.299999 45.799999) (width 0.5) (layer F.Cu) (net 2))
 (segment (start 63.624003 45.699999) (end 62.399999 45.699999) (width 0.5) (layer F.Cu) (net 2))
 (segment (start 65.024002 44.3) (end 63.624003 45.699999) (width 0.5) (layer F.Cu) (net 2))
 (segment (start 65.6 44.3) (end 65.024002 44.3) (width 0.5) (layer F.Cu) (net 2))
 (segment (start 82 45.24) (end 81.9 45.14) (width 0.5) (layer F.Cu) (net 2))
 (segment (start 63.6 57.14) (end 63.7 57.24) (width 0.5) (layer F.Cu) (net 2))
 (segment (start 63.6 54.62) (end 63.6 57.14) (width 0.5) (layer F.Cu) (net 2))
 (segment (start 62.3 58.64) (end 63.7 57.24) (width 0.5) (layer B.Cu) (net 2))
 (segment (start 62.3 69.59137) (end 62.3 58.64) (width 0.5) (layer B.Cu) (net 2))
 (segment (start 65.10863 72.4) (end 62.3 69.59137) (width 0.5) (layer B.Cu) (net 2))
 (segment (start 66.24 72.4) (end 65.10863 72.4) (width 0.5) (layer B.Cu) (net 2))
 (segment (start 67.039999 71.600001) (end 69.529999 71.600001) (width 0.5) (layer F.Cu) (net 2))
 (segment (start 69.529999 71.600001) (end 70.680001 70.449999) (width 0.5) (layer F.Cu) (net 2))
 (segment (start 70.680001 70.449999) (end 71.53 69.6) (width 0.5) (layer F.Cu) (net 2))
 (segment (start 66.24 72.4) (end 67.039999 71.600001) (width 0.5) (layer F.Cu) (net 2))
 (segment (start 86.52 68.38) (end 86.52 65.84) (width 0.5) (layer B.Cu) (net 2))
 (segment (start 78.9 68.38) (end 78.9 65.84) (width 0.5) (layer B.Cu) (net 2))
 (segment (start 80.03137 65.84) (end 86.52 65.84) (width 0.5) (layer F.Cu) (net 2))
 (segment (start 78.9 65.84) (end 80.03137 65.84) (width 0.5) (layer F.Cu) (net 2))
 (segment (start 85.799999 46.039999) (end 85 45.24) (width 0.5) (layer F.Cu) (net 2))
 (segment (start 87.820001 48.060001) (end 85.799999 46.039999) (width 0.5) (layer F.Cu) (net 2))
 (segment (start 87.820001 63.924001) (end 87.820001 48.060001) (width 0.5) (layer F.Cu) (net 2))
 (segment (start 86.52 65.224002) (end 87.820001 63.924001) (width 0.5) (layer F.Cu) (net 2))
 (segment (start 86.52 65.84) (end 86.52 65.224002) (width 0.5) (layer F.Cu) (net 2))
 (segment (start 85 45.24) (end 82 45.24) (width 0.5) (layer F.Cu) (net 2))
 (segment (start 80.4 40.14) (end 78.9 40.14) (width 0.5) (layer F.Cu) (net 2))
 (segment (start 82 41.74) (end 80.4 40.14) (width 0.5) (layer F.Cu) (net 2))
 (segment (start 82 45.24) (end 82 41.74) (width 0.5) (layer F.Cu) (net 2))
 (segment (start 71.4883 43.0481) (end 71.4883 44.4481) (width 0.5) (layer B.Cu) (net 2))
 (segment (start 74.3964 40.14) (end 71.4883 43.0481) (width 0.5) (layer B.Cu) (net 2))
 (segment (start 78.9 40.14) (end 74.3964 40.14) (width 0.5) (layer B.Cu) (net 2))
 (segment (start 73.220001 70.449999) (end 74.07 69.6) (width 0.25) (layer F.Cu) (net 16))
 (segment (start 66.024999 73.575001) (end 66.804001 73.575001) (width 0.25) (layer F.Cu) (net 16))
 (segment (start 64.7 73.6) (end 66 73.6) (width 0.25) (layer F.Cu) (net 16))
 (segment (start 62.500011 71.400011) (end 64.7 73.6) (width 0.25) (layer F.Cu) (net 16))
 (segment (start 66.424999 57.375001) (end 62.500011 61.299989) (width 0.25) (layer F.Cu) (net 16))
 (segment (start 66.424999 56.909999) (end 66.424999 57.375001) (width 0.25) (layer F.Cu) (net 16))
 (segment (start 66.975001 56.824999) (end 66.509999 56.824999) (width 0.25) (layer F.Cu) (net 16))
 (segment (start 67.099991 56.651467) (end 67.099991 56.700009) (width 0.25) (layer F.Cu) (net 16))
 (segment (start 66 73.6) (end 66.024999 73.575001) (width 0.25) (layer F.Cu) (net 16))
 (segment (start 71.37 72.3) (end 73.220001 70.449999) (width 0.25) (layer F.Cu) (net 16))
 (segment (start 68.079002 72.3) (end 71.37 72.3) (width 0.25) (layer F.Cu) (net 16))
 (segment (start 66.509999 56.824999) (end 66.424999 56.909999) (width 0.25) (layer F.Cu) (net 16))
 (segment (start 62.500011 61.299989) (end 62.500011 71.400011) (width 0.25) (layer F.Cu) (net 16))
 (segment (start 76.3 48.13137) (end 71.036371 53.394999) (width 0.25) (layer F.Cu) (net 16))
 (segment (start 67.365001 54.121997) (end 67.365001 56.386457) (width 0.25) (layer F.Cu) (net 16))
 (segment (start 71.036371 53.394999) (end 68.091999 53.394999) (width 0.25) (layer F.Cu) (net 16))
 (segment (start 68.091999 53.394999) (end 67.365001 54.121997) (width 0.25) (layer F.Cu) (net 16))
 (segment (start 66.804001 73.575001) (end 68.079002 72.3) (width 0.25) (layer F.Cu) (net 16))
 (segment (start 67.365001 56.386457) (end 67.099991 56.651467) (width 0.25) (layer F.Cu) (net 16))
 (segment (start 76.3 47) (end 76.3 48.13137) (width 0.25) (layer F.Cu) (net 16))
 (segment (start 67.099991 56.700009) (end 66.975001 56.824999) (width 0.25) (layer F.Cu) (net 16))
 (segment (start 77.614999 45.774999) (end 75.711999 45.774999) (width 0.25) (layer F.Cu) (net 15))
 (segment (start 73.35999 72.85001) (end 75.760001 70.449999) (width 0.25) (layer F.Cu) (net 15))
 (segment (start 64.914999 54.031999) (end 64.914999 56.641997) (width 0.25) (layer F.Cu) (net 15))
 (segment (start 78.84 47) (end 77.614999 45.774999) (width 0.25) (layer F.Cu) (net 15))
 (segment (start 70.808551 52.844989) (end 66.102009 52.844989) (width 0.25) (layer F.Cu) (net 15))
 (segment (start 64.9 58.122169) (end 62 61.022169) (width 0.25) (layer F.Cu) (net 15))
 (segment (start 75.711999 45.774999) (end 75.074999 46.411999) (width 0.25) (layer F.Cu) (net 15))
 (segment (start 68.306823 72.85001) (end 73.35999 72.85001) (width 0.25) (layer F.Cu) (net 15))
 (segment (start 75.074999 46.411999) (end 75.074999 48.578541) (width 0.25) (layer F.Cu) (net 15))
 (segment (start 75.074999 48.578541) (end 70.808551 52.844989) (width 0.25) (layer F.Cu) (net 15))
 (segment (start 62 61.022169) (end 62 71.677831) (width 0.25) (layer F.Cu) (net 15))
 (segment (start 66.102009 52.844989) (end 64.914999 54.031999) (width 0.25) (layer F.Cu) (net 15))
 (segment (start 64.9 57.7) (end 64.9 58.122169) (width 0.25) (layer F.Cu) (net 15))
 (segment (start 64.914999 56.641997) (end 64.925001 56.651999) (width 0.25) (layer F.Cu) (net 15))
 (segment (start 62 71.677831) (end 64.472179 74.15001) (width 0.25) (layer F.Cu) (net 15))
 (segment (start 64.925001 56.651999) (end 64.925001 57.674999) (width 0.25) (layer F.Cu) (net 15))
 (segment (start 64.925001 57.674999) (end 64.9 57.7) (width 0.25) (layer F.Cu) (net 15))
 (segment (start 64.472179 74.15001) (end 67.006823 74.15001) (width 0.25) (layer F.Cu) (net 15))
 (segment (start 67.006823 74.15001) (end 68.306823 72.85001) (width 0.25) (layer F.Cu) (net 15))
 (segment (start 75.760001 70.449999) (end 76.61 69.6) (width 0.25) (layer F.Cu) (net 15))
 (segment (start 76.9 63.3) (end 78.9 63.3) (width 0.5) (layer F.Cu) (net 8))
 (segment (start 75.24 61.64) (end 76.9 63.3) (width 0.5) (layer F.Cu) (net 8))
 (segment (start 75.24 61.6) (end 75.24 61.64) (width 0.5) (layer F.Cu) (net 8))
 (segment (start 78.100001 70.120001) (end 78.9 70.92) (width 0.25) (layer F.Cu) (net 10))
 (segment (start 78.100001 69.276999) (end 78.100001 70.120001) (width 0.25) (layer F.Cu) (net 10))
 (segment (start 77.198001 68.374999) (end 78.100001 69.276999) (width 0.25) (layer F.Cu) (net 10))
 (segment (start 76.374999 68.374999) (end 77.198001 68.374999) (width 0.25) (layer F.Cu) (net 10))
 (segment (start 73.474999 65.474999) (end 76.374999 68.374999) (width 0.25) (layer F.Cu) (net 10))
 (segment (start 73.474999 63.474999) (end 73.474999 65.474999) (width 0.25) (layer F.Cu) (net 10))
 (segment (start 72.7 62.7) (end 73.474999 63.474999) (width 0.25) (layer F.Cu) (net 10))
 (segment (start 72.7 61.6) (end 72.7 62.7) (width 0.25) (layer F.Cu) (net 10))
 (segment (start 72.1364 37.6) (end 71.4883 38.2481) (width 0.5) (layer B.Cu) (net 3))
 (segment (start 78.9 37.6) (end 72.1364 37.6) (width 0.5) (layer B.Cu) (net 3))
 (segment (start 80.40001 56.71999) (end 79.699999 57.420001) (width 0.5) (layer B.Cu) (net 3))
 (segment (start 80.40001 39.05251) (end 80.40001 56.71999) (width 0.5) (layer B.Cu) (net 3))
 (segment (start 79.699999 57.420001) (end 78.9 58.22) (width 0.5) (layer B.Cu) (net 3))
 (segment (start 78.9475 37.6) (end 80.40001 39.05251) (width 0.5) (layer B.Cu) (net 3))
 (segment (start 78.9 37.6) (end 78.9475 37.6) (width 0.5) (layer B.Cu) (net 3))
 (segment (start 66.45 68.4) (end 66.45 69.6) (width 0.35) (layer B.Cu) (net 9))
 (segment (start 76.834003 68.324999) (end 66.525001 68.324999) (width 0.35) (layer B.Cu) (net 9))
 (segment (start 77.695001 67.464001) (end 76.834003 68.324999) (width 0.35) (layer B.Cu) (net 9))
 (segment (start 77.695001 66.448003) (end 77.695001 67.464001) (width 0.35) (layer B.Cu) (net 9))
 (segment (start 77.674999 66.428001) (end 77.695001 66.448003) (width 0.35) (layer B.Cu) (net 9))
 (segment (start 77.674999 65.225001) (end 77.674999 66.428001) (width 0.35) (layer B.Cu) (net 9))
 (segment (start 78.374999 64.525001) (end 77.674999 65.225001) (width 0.35) (layer B.Cu) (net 9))
 (segment (start 66.525001 68.324999) (end 66.45 68.4) (width 0.35) (layer B.Cu) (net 9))
 (segment (start 85.294999 64.525001) (end 78.374999 64.525001) (width 0.35) (layer B.Cu) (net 9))
 (segment (start 86.52 63.3) (end 85.294999 64.525001) (width 0.35) (layer B.Cu) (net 9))
 (segment (start 85.38863 70.92) (end 86.52 70.92) (width 0.35) (layer B.Cu) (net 7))
 (segment (start 82.40117 70.92) (end 85.38863 70.92) (width 0.35) (layer B.Cu) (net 7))
 (segment (start 77.341997 71.174999) (end 78.311999 72.145001) (width 0.35) (layer B.Cu) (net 7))
 (segment (start 70.564999 71.174999) (end 77.341997 71.174999) (width 0.35) (layer B.Cu) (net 7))
 (segment (start 81.176169 72.145001) (end 82.40117 70.92) (width 0.35) (layer B.Cu) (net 7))
 (segment (start 68.99 69.6) (end 70.564999 71.174999) (width 0.35) (layer B.Cu) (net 7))
 (segment (start 78.311999 72.145001) (end 81.176169 72.145001) (width 0.35) (layer B.Cu) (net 7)))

